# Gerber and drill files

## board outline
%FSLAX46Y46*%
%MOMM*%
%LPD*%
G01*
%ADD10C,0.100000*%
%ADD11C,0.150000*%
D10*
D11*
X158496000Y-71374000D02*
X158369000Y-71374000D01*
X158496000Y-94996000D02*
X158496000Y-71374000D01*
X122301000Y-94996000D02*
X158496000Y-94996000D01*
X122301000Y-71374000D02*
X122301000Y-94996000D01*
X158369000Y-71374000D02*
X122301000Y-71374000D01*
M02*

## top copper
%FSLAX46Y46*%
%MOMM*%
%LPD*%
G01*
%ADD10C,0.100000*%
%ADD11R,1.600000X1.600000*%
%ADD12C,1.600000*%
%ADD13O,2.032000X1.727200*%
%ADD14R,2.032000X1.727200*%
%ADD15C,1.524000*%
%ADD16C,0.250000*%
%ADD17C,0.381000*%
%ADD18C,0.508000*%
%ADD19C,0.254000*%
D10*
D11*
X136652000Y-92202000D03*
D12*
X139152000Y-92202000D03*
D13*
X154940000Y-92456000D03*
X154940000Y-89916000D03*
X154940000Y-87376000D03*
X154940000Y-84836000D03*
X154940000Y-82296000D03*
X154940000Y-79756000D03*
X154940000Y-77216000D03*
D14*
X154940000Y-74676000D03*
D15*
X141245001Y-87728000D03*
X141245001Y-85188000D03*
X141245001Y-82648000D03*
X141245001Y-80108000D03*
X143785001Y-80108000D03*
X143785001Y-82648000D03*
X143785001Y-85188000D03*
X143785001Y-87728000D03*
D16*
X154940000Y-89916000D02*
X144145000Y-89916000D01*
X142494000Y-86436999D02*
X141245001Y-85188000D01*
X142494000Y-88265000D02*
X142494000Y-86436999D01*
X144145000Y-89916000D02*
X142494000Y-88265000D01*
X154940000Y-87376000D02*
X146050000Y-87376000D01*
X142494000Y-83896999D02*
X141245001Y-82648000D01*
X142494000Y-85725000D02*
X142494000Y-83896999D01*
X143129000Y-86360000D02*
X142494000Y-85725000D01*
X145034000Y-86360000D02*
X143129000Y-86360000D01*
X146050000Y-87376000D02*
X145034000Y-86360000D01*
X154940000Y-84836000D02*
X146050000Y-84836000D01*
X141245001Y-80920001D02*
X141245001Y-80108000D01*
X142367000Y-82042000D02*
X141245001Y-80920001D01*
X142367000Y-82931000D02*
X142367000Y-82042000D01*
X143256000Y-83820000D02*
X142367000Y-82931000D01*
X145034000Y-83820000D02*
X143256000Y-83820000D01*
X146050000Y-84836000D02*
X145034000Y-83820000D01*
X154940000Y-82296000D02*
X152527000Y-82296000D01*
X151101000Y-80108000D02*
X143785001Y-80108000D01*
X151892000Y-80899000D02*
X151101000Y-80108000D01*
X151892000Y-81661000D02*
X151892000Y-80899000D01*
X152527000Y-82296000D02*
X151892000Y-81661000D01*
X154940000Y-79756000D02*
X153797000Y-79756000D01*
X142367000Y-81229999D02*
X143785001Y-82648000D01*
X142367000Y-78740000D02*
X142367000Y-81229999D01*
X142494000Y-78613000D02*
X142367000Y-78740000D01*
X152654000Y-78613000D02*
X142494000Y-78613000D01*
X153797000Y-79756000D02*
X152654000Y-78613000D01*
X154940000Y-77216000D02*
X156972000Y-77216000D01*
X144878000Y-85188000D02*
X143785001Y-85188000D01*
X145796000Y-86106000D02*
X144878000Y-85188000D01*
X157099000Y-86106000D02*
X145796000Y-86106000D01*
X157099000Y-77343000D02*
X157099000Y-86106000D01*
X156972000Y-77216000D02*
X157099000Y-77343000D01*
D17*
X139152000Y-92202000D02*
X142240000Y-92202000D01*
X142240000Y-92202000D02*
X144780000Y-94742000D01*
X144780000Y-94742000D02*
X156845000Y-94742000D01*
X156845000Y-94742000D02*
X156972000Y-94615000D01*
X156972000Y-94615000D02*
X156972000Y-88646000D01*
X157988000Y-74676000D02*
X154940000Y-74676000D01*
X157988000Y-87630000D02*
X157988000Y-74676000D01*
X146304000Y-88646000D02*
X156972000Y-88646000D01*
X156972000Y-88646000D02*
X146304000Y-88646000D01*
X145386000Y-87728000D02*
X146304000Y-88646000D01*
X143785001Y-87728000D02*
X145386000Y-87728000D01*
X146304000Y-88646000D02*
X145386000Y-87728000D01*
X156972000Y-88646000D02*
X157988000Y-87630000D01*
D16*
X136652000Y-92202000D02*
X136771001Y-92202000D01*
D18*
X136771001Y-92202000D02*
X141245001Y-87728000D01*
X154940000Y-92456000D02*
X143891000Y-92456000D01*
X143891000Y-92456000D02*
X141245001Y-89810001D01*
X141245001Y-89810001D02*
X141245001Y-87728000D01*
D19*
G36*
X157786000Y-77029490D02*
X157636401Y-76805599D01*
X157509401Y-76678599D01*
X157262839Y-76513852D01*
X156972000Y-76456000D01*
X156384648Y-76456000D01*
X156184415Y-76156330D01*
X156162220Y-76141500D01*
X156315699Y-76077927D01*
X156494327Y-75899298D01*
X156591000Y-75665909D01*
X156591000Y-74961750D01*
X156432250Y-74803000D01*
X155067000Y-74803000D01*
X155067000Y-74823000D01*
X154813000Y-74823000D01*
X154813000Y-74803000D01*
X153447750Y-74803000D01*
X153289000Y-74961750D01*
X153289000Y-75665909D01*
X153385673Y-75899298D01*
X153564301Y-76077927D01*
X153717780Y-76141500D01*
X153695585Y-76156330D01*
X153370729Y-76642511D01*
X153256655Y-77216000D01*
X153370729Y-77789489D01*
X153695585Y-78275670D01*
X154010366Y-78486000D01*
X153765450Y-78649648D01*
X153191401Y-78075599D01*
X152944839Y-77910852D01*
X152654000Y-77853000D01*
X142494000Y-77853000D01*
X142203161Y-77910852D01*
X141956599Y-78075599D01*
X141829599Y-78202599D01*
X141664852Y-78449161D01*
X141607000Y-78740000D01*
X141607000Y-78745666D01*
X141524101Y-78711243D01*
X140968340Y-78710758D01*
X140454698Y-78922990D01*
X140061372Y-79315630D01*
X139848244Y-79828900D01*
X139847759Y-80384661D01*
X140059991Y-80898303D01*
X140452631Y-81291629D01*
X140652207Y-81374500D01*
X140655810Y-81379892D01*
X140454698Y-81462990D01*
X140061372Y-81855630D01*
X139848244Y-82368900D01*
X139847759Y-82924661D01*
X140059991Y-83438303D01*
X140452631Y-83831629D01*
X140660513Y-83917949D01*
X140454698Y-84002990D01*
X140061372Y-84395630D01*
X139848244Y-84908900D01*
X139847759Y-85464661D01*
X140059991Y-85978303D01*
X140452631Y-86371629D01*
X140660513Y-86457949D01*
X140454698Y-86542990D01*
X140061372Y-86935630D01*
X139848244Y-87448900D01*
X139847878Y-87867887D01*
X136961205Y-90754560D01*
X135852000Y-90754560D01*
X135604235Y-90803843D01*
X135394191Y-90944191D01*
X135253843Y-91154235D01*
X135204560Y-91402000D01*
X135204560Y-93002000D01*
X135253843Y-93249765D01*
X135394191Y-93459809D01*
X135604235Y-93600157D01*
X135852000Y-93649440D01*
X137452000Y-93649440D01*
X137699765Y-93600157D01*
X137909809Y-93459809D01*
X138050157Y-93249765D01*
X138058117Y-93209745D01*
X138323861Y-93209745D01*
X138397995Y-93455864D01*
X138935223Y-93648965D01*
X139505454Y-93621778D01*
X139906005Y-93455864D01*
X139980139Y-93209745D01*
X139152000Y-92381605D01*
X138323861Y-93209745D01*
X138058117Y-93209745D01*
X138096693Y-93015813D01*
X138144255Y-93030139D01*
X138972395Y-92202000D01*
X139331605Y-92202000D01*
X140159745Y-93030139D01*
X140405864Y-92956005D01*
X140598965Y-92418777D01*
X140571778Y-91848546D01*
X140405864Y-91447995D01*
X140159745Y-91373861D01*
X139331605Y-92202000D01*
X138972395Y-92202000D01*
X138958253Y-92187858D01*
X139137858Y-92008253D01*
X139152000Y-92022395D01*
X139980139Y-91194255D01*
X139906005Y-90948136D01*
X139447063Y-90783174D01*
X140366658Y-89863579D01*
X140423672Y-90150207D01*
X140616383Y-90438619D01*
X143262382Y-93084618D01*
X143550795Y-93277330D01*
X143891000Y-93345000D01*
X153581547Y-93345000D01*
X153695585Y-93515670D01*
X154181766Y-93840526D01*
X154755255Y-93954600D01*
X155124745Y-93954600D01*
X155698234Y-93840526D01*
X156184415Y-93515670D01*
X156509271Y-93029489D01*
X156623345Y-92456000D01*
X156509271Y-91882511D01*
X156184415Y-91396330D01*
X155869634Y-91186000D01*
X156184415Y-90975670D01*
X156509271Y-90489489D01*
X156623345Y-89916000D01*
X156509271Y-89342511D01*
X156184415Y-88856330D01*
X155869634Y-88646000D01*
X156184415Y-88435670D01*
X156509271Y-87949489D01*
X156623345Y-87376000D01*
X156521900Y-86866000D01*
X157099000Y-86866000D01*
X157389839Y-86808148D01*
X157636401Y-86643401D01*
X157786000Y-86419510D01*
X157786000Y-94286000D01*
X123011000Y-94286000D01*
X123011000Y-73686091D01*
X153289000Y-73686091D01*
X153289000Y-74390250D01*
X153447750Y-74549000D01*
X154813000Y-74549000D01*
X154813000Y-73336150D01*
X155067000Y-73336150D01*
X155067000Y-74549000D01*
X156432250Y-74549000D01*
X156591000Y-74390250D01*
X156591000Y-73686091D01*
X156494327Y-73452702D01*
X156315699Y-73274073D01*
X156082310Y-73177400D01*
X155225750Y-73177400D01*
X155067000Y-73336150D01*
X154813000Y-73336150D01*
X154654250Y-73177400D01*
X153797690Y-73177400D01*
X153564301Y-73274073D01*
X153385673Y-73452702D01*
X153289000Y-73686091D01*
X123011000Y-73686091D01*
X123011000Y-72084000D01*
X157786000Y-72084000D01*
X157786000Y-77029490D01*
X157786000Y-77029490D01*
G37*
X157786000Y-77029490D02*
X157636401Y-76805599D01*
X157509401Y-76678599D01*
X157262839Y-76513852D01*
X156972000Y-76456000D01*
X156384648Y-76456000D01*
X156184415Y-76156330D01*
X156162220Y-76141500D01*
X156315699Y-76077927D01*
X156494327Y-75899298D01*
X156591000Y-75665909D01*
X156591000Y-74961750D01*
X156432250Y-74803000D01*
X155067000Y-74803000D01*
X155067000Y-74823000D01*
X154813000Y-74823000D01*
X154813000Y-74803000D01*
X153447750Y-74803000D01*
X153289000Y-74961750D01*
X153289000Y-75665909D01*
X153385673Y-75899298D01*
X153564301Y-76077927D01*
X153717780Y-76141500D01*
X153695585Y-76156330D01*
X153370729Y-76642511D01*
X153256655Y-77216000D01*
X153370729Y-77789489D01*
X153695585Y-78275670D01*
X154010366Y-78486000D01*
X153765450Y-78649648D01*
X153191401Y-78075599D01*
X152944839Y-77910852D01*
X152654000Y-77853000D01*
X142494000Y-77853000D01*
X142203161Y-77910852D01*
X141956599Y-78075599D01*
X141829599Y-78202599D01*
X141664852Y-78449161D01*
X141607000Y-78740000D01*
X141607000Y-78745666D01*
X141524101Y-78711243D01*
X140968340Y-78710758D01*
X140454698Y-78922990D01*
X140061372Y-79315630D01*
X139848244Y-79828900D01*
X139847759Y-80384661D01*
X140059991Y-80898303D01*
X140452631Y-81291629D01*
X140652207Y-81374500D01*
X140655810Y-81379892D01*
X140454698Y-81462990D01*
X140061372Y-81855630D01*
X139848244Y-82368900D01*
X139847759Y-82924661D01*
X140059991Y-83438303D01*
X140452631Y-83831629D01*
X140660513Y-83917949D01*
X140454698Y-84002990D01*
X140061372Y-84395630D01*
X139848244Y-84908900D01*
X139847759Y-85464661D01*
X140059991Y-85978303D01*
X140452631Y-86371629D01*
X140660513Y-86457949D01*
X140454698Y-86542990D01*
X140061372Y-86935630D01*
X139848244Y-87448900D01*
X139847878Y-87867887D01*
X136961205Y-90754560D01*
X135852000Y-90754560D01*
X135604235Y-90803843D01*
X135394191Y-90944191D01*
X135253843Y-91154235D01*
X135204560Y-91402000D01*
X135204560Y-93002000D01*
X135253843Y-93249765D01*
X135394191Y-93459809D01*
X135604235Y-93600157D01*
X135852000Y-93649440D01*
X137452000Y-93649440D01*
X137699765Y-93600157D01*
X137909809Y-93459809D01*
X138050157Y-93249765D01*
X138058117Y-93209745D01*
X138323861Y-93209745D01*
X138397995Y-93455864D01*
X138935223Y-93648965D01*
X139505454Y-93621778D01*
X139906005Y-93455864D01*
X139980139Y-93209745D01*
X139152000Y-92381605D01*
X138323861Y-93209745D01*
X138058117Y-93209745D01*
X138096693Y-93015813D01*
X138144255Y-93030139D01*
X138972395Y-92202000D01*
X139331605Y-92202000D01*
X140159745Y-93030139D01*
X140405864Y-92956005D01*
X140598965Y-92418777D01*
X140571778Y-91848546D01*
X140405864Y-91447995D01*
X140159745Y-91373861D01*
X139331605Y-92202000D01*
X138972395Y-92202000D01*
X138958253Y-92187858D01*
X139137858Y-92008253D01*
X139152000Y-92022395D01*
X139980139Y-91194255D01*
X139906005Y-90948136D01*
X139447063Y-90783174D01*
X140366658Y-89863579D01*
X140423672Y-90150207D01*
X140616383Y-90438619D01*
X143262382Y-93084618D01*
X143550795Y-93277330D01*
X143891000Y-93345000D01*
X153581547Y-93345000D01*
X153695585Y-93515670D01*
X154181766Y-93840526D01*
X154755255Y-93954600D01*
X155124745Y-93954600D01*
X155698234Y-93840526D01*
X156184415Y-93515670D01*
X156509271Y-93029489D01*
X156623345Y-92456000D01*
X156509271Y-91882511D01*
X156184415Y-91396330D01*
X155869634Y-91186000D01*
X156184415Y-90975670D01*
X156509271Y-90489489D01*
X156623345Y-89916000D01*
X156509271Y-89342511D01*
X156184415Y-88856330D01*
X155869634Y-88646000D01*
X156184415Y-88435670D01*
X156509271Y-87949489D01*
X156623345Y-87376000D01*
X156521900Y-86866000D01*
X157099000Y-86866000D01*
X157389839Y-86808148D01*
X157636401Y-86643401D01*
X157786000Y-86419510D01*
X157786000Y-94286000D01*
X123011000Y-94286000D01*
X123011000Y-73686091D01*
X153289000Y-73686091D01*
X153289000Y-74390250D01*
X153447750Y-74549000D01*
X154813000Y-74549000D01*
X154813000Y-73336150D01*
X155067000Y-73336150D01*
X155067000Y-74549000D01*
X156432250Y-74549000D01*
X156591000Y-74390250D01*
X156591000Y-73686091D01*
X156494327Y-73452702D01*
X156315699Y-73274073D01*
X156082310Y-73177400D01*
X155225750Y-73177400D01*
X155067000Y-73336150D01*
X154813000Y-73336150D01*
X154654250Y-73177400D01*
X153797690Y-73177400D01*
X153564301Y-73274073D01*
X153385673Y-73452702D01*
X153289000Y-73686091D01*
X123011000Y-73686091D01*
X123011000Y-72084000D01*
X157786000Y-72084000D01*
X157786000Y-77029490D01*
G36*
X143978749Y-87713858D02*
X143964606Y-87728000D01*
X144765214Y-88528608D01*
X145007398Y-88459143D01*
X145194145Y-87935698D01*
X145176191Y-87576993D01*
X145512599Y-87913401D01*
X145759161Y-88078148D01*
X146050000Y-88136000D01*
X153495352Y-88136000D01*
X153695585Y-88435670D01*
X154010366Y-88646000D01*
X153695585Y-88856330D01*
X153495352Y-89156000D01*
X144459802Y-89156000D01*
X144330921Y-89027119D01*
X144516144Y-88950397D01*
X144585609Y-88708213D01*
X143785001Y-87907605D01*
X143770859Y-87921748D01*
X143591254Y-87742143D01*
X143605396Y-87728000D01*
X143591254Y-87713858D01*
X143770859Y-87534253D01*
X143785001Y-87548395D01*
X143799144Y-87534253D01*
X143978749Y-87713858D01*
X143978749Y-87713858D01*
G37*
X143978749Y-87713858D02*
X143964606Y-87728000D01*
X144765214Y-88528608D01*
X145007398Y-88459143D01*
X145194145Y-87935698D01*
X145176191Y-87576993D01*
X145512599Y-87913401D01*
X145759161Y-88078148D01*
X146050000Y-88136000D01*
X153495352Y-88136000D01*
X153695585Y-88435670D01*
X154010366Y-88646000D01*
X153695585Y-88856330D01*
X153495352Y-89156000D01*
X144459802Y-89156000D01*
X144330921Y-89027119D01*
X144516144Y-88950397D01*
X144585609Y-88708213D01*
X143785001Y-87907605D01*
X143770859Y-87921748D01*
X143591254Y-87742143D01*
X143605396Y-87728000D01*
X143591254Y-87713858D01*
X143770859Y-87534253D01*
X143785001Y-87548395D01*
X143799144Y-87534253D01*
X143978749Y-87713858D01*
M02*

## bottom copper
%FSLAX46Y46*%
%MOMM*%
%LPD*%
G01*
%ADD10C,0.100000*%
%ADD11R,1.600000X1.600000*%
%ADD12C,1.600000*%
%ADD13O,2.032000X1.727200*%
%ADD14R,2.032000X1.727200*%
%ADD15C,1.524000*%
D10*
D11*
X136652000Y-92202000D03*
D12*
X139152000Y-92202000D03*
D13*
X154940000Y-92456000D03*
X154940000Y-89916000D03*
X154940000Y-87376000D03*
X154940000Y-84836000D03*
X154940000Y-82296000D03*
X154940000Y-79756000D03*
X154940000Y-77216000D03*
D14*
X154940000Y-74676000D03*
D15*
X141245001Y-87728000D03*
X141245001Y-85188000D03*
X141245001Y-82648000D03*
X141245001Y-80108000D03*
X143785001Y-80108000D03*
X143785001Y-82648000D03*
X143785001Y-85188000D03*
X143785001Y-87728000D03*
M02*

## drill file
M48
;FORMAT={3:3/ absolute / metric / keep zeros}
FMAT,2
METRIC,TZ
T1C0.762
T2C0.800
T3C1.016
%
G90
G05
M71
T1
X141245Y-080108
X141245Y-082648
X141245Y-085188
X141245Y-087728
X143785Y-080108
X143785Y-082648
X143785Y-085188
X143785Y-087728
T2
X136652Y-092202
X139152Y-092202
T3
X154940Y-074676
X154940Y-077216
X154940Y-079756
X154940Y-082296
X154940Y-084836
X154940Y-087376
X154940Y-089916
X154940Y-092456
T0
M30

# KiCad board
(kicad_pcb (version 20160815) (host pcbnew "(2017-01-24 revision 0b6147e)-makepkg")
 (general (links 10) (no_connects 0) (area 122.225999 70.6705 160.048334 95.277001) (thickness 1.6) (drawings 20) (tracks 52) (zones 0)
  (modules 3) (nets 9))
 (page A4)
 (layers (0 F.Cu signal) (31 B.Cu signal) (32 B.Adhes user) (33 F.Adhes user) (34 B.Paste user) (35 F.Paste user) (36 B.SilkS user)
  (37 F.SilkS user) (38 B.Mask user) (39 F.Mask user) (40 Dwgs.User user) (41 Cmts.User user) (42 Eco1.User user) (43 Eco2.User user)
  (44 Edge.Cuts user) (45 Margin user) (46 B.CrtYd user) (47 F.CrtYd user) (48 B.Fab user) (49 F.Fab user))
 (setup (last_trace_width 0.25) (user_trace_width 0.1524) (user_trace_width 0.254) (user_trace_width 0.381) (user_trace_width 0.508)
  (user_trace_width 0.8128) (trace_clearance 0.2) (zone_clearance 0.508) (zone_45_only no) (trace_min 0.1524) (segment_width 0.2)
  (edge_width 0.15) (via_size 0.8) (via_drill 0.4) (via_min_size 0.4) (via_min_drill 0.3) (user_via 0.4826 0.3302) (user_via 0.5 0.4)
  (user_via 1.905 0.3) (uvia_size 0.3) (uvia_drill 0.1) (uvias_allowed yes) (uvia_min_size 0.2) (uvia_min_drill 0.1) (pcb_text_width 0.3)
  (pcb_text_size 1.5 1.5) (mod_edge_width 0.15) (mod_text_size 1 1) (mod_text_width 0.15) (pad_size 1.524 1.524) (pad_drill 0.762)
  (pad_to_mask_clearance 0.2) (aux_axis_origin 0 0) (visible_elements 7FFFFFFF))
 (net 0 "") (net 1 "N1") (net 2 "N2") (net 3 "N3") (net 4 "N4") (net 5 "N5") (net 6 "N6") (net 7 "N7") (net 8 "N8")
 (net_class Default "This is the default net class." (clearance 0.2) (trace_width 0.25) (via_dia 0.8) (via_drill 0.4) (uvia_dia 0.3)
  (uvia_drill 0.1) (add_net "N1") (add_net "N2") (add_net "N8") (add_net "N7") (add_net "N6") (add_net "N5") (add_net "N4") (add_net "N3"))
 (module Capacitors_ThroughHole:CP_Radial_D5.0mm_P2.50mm (layer F.Cu) (at 136.652 92.202)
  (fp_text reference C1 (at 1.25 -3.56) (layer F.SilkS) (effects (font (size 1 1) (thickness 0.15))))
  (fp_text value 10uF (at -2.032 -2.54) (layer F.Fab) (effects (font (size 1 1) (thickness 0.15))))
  (pad 1 thru_hole rect (at 0 0) (size 1.6 1.6) (drill 0.8) (layers *.Cu *.Mask) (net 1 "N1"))
  (pad 2 thru_hole circle (at 2.5 0) (size 1.6 1.6) (drill 0.8) (layers *.Cu *.Mask) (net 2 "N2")))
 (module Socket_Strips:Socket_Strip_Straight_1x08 (layer F.Cu) (at 154.94 74.676 270)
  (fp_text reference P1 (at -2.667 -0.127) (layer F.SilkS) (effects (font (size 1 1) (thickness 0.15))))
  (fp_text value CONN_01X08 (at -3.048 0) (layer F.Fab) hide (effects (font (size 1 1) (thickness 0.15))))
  (pad 8 thru_hole oval (at 17.78 0 270) (size 1.7272 2.032) (drill 1.016) (layers *.Cu *.Mask) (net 1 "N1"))
  (pad 7 thru_hole oval (at 15.24 0 270) (size 1.7272 2.032) (drill 1.016) (layers *.Cu *.Mask) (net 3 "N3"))
  (pad 6 thru_hole oval (at 12.7 0 270) (size 1.7272 2.032) (drill 1.016) (layers *.Cu *.Mask) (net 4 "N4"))
  (pad 5 thru_hole oval (at 10.16 0 270) (size 1.7272 2.032) (drill 1.016) (layers *.Cu *.Mask) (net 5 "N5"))
  (pad 4 thru_hole oval (at 7.62 0 270) (size 1.7272 2.032) (drill 1.016) (layers *.Cu *.Mask) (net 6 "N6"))
  (pad 3 thru_hole oval (at 5.08 0 270) (size 1.7272 2.032) (drill 1.016) (layers *.Cu *.Mask) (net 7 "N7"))
  (pad 2 thru_hole oval (at 2.54 0 270) (size 1.7272 2.032) (drill 1.016) (layers *.Cu *.Mask) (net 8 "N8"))
  (pad 1 thru_hole rect (at 0 0 270) (size 1.7272 2.032) (drill 1.016) (layers *.Cu *.Mask) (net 2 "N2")))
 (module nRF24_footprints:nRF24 (layer F.Cu) (at 133.625001 77.568)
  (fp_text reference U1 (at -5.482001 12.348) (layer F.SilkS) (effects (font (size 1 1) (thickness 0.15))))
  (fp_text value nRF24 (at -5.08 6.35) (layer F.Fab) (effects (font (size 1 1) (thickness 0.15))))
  (pad 7 thru_hole circle (at 7.62 10.16) (size 1.524 1.524) (drill 0.762) (layers *.Cu *.Mask) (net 1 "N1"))
  (pad 6 thru_hole circle (at 7.62 7.62) (size 1.524 1.524) (drill 0.762) (layers *.Cu *.Mask) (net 3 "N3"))
  (pad 5 thru_hole circle (at 7.62 5.08) (size 1.524 1.524) (drill 0.762) (layers *.Cu *.Mask) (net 4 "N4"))
  (pad 4 thru_hole circle (at 7.62 2.54) (size 1.524 1.524) (drill 0.762) (layers *.Cu *.Mask) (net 5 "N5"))
  (pad 3 thru_hole circle (at 10.16 2.54) (size 1.524 1.524) (drill 0.762) (layers *.Cu *.Mask) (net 6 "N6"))
  (pad 2 thru_hole circle (at 10.16 5.08) (size 1.524 1.524) (drill 0.762) (layers *.Cu *.Mask) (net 7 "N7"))
  (pad 1 thru_hole circle (at 10.16 7.62) (size 1.524 1.524) (drill 0.762) (layers *.Cu *.Mask) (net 8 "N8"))
  (pad 0 thru_hole circle (at 10.16 10.16) (size 1.524 1.524) (drill 0.762) (layers *.Cu *.Mask) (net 2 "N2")))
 (gr_line (start 158.496 71.374) (end 158.369 71.374) (angle 90) (layer Edge.Cuts) (width 0.15))
 (gr_line (start 158.496 94.996) (end 158.496 71.374) (angle 90) (layer Edge.Cuts) (width 0.15))
 (gr_line (start 122.301 94.996) (end 158.496 94.996) (angle 90) (layer Edge.Cuts) (width 0.15))
 (gr_line (start 122.301 71.374) (end 122.301 94.996) (angle 90) (layer Edge.Cuts) (width 0.15))
 (gr_line (start 158.369 71.374) (end 122.301 71.374) (angle 90) (layer Edge.Cuts) (width 0.15))
 (segment (start 154.94 89.916) (end 144.145 89.916) (width 0.25) (layer F.Cu) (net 3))
 (segment (start 142.494 86.436999) (end 141.245001 85.188) (width 0.25) (layer F.Cu) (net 3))
 (segment (start 142.494 88.265) (end 142.494 86.436999) (width 0.25) (layer F.Cu) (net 3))
 (segment (start 144.145 89.916) (end 142.494 88.265) (width 0.25) (layer F.Cu) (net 3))
 (segment (start 154.94 87.376) (end 146.05 87.376) (width 0.25) (layer F.Cu) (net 4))
 (segment (start 142.494 83.896999) (end 141.245001 82.648) (width 0.25) (layer F.Cu) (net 4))
 (segment (start 142.494 85.725) (end 142.494 83.896999) (width 0.25) (layer F.Cu) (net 4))
 (segment (start 143.129 86.36) (end 142.494 85.725) (width 0.25) (layer F.Cu) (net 4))
 (segment (start 145.034 86.36) (end 143.129 86.36) (width 0.25) (layer F.Cu) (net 4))
 (segment (start 146.05 87.376) (end 145.034 86.36) (width 0.25) (layer F.Cu) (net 4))
 (segment (start 154.94 84.836) (end 146.05 84.836) (width 0.25) (layer F.Cu) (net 5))
 (segment (start 141.245001 80.920001) (end 141.245001 80.108) (width 0.25) (layer F.Cu) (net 5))
 (segment (start 142.367 82.042) (end 141.245001 80.920001) (width 0.25) (layer F.Cu) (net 5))
 (segment (start 142.367 82.931) (end 142.367 82.042) (width 0.25) (layer F.Cu) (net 5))
 (segment (start 143.256 83.82) (end 142.367 82.931) (width 0.25) (layer F.Cu) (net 5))
 (segment (start 145.034 83.82) (end 143.256 83.82) (width 0.25) (layer F.Cu) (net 5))
 (segment (start 146.05 84.836) (end 145.034 83.82) (width 0.25) (layer F.Cu) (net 5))
 (segment (start 154.94 82.296) (end 152.527 82.296) (width 0.25) (layer F.Cu) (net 6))
 (segment (start 151.101 80.108) (end 143.785001 80.108) (width 0.25) (layer F.Cu) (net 6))
 (segment (start 151.892 80.899) (end 151.101 80.108) (width 0.25) (layer F.Cu) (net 6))
 (segment (start 151.892 81.661) (end 151.892 80.899) (width 0.25) (layer F.Cu) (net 6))
 (segment (start 152.527 82.296) (end 151.892 81.661) (width 0.25) (layer F.Cu) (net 6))
 (segment (start 154.94 79.756) (end 153.797 79.756) (width 0.25) (layer F.Cu) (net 7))
 (segment (start 142.367 81.229999) (end 143.785001 82.648) (width 0.25) (layer F.Cu) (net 7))
 (segment (start 142.367 78.74) (end 142.367 81.229999) (width 0.25) (layer F.Cu) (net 7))
 (segment (start 142.494 78.613) (end 142.367 78.74) (width 0.25) (layer F.Cu) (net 7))
 (segment (start 152.654 78.613) (end 142.494 78.613) (width 0.25) (layer F.Cu) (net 7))
 (segment (start 153.797 79.756) (end 152.654 78.613) (width 0.25) (layer F.Cu) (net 7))
 (segment (start 154.94 77.216) (end 156.972 77.216) (width 0.25) (layer F.Cu) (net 8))
 (segment (start 144.878 85.188) (end 143.785001 85.188) (width 0.25) (layer F.Cu) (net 8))
 (segment (start 145.796 86.106) (end 144.878 85.188) (width 0.25) (layer F.Cu) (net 8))
 (segment (start 157.099 86.106) (end 145.796 86.106) (width 0.25) (layer F.Cu) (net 8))
 (segment (start 157.099 77.343) (end 157.099 86.106) (width 0.25) (layer F.Cu) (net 8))
 (segment (start 156.972 77.216) (end 157.099 77.343) (width 0.25) (layer F.Cu) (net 8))
 (segment (start 139.152 92.202) (end 142.24 92.202) (width 0.381) (layer F.Cu) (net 2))
 (segment (start 142.24 92.202) (end 144.78 94.742) (width 0.381) (layer F.Cu) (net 2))
 (segment (start 144.78 94.742) (end 156.845 94.742) (width 0.381) (layer F.Cu) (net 2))
 (segment (start 156.845 94.742) (end 156.972 94.615) (width 0.381) (layer F.Cu) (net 2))
 (segment (start 156.972 94.615) (end 156.972 88.646) (width 0.381) (layer F.Cu) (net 2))
 (segment (start 157.988 74.676) (end 154.94 74.676) (width 0.381) (layer F.Cu) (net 2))
 (segment (start 157.988 87.63) (end 157.988 74.676) (width 0.381) (layer F.Cu) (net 2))
 (segment (start 146.304 88.646) (end 156.972 88.646) (width 0.381) (layer F.Cu) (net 2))
 (segment (start 156.972 88.646) (end 146.304 88.646) (width 0.381) (layer F.Cu) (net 2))
 (segment (start 145.386 87.728) (end 146.304 88.646) (width 0.381) (layer F.Cu) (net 2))
 (segment (start 143.785001 87.728) (end 145.386 87.728) (width 0.381) (layer F.Cu) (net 2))
 (segment (start 146.304 88.646) (end 145.386 87.728) (width 0.381) (layer F.Cu) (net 2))
 (segment (start 156.972 88.646) (end 157.988 87.63) (width 0.381) (layer F.Cu) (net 2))
 (segment (start 136.652 92.202) (end 136.771001 92.202) (width 0.25) (layer F.Cu) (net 1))
 (segment (start 136.771001 92.202) (end 141.245001 87.728) (width 0.508) (layer F.Cu) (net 1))
 (segment (start 154.94 92.456) (end 143.891 92.456) (width 0.508) (layer F.Cu) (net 1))
 (segment (start 143.891 92.456) (end 141.245001 89.810001) (width 0.508) (layer F.Cu) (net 1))
 (segment (start 141.245001 89.810001) (end 141.245001 87.728) (width 0.508) (layer F.Cu) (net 1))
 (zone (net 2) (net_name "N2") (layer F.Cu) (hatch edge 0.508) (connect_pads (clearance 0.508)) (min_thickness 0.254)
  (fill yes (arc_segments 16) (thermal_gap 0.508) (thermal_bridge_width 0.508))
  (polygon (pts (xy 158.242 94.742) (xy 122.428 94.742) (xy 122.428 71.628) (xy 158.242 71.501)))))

